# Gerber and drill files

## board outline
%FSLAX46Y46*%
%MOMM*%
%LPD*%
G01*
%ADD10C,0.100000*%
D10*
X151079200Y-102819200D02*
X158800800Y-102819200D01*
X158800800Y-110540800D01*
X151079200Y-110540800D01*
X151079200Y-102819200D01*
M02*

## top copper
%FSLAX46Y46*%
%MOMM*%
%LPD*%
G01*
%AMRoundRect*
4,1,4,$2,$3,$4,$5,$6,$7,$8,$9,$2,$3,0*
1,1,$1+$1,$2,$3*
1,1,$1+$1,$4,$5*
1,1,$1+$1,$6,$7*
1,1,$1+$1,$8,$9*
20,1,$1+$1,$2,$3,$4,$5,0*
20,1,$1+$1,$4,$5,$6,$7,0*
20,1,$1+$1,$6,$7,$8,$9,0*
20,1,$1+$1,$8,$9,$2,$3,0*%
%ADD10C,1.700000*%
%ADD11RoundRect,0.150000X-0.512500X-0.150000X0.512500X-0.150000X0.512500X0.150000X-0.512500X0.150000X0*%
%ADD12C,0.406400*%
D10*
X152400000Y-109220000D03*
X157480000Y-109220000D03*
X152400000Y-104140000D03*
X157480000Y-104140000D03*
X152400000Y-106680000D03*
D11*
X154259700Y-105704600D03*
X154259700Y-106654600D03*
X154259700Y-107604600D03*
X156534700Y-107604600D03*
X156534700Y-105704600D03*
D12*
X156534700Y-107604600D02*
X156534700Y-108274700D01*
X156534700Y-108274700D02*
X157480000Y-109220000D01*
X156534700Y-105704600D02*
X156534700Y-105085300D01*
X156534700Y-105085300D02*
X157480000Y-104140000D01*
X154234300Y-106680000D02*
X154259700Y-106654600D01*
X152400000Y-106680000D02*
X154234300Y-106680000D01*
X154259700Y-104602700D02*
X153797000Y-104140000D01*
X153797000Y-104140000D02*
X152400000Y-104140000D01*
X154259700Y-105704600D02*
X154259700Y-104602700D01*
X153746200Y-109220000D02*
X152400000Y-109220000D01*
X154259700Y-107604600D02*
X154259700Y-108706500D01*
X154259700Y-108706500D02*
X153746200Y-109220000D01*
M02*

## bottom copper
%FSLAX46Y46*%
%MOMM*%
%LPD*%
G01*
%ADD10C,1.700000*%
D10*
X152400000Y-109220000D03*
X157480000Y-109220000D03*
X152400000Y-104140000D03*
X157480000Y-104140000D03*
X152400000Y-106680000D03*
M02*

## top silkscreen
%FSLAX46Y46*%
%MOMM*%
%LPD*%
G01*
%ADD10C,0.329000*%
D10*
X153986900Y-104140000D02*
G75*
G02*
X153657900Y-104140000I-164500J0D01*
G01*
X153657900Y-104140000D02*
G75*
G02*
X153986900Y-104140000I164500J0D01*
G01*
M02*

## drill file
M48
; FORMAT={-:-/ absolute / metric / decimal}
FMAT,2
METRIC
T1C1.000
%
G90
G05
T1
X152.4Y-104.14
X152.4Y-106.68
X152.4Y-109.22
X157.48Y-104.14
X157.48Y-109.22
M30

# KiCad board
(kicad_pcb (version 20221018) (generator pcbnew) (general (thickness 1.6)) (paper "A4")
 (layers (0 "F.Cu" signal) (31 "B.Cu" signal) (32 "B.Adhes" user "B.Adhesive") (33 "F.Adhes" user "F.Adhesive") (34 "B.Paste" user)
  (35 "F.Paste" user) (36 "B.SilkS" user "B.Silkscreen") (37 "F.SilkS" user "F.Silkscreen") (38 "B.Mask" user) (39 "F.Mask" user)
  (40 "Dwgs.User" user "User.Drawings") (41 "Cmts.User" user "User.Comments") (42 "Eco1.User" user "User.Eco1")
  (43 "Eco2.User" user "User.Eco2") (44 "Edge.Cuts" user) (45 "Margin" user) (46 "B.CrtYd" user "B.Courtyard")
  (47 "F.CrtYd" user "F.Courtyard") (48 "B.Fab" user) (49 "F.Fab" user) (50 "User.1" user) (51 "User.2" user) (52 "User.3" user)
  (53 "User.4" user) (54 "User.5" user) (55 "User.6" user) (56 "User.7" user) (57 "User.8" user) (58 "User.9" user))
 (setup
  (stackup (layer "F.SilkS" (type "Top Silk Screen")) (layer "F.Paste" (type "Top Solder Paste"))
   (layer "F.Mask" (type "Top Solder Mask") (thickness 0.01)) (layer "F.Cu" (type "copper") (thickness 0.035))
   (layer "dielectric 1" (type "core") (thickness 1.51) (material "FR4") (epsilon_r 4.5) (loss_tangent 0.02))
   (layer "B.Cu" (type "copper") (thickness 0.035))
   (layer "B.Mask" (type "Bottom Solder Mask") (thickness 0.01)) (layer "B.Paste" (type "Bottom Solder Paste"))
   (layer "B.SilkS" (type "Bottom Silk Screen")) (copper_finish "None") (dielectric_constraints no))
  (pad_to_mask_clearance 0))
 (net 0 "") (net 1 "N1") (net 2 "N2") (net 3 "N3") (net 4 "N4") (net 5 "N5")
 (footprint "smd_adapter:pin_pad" (layer "F.Cu") (at 152.4 109.22)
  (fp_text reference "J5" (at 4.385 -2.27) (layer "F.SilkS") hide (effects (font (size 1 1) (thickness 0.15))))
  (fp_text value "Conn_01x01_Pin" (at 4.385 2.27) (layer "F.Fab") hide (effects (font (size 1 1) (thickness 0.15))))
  (pad "1" thru_hole circle (at 0 0) (size 1.7 1.7) (drill 1) (layers "*.Cu" "*.Mask") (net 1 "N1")))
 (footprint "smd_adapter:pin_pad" (layer "F.Cu") (at 157.48 109.22)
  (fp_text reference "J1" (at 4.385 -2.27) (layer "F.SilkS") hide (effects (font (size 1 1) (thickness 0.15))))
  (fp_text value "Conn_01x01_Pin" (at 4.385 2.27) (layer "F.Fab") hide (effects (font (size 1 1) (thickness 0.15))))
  (pad "1" thru_hole circle (at 0 0) (size 1.7 1.7) (drill 1) (layers "*.Cu" "*.Mask") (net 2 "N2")))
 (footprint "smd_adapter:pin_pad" (layer "F.Cu") (at 152.4 104.14)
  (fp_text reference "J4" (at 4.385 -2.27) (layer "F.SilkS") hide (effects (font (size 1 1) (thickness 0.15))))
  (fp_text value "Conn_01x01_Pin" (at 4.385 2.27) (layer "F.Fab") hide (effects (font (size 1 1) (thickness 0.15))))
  (pad "1" thru_hole circle (at 0 0) (size 1.7 1.7) (drill 1) (layers "*.Cu" "*.Mask") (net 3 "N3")))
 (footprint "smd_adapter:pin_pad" (layer "F.Cu") (at 157.48 104.14)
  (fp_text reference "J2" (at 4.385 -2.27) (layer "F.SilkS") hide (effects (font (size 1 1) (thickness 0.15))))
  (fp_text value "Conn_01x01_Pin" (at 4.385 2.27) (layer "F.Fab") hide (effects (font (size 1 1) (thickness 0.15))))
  (pad "1" thru_hole circle (at 0 0) (size 1.7 1.7) (drill 1) (layers "*.Cu" "*.Mask") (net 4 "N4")))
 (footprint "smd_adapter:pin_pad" (layer "F.Cu") (at 152.4 106.68)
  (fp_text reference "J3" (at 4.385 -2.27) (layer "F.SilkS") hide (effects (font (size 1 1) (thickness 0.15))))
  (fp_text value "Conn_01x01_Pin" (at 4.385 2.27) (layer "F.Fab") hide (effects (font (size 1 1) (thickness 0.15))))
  (pad "1" thru_hole circle (at 0 0) (size 1.7 1.7) (drill 1) (layers "*.Cu" "*.Mask") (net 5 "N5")))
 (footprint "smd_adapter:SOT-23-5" (layer "F.Cu") (at 155.3972 106.6546)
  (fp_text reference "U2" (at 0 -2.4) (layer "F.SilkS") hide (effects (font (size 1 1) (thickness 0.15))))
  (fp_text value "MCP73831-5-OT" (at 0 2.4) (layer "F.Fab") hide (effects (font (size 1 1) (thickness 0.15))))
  (pad "1" smd roundrect (at -1.1375 -0.95) (size 1.325 0.6) (layers "F.Cu" "F.Paste" "F.Mask") (roundrect_rratio 0.25) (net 3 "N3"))
  (pad "2" smd roundrect (at -1.1375 0) (size 1.325 0.6) (layers "F.Cu" "F.Paste" "F.Mask") (roundrect_rratio 0.25) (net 5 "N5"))
  (pad "3" smd roundrect (at -1.1375 0.95) (size 1.325 0.6) (layers "F.Cu" "F.Paste" "F.Mask") (roundrect_rratio 0.25) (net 1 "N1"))
  (pad "4" smd roundrect (at 1.1375 0.95) (size 1.325 0.6) (layers "F.Cu" "F.Paste" "F.Mask") (roundrect_rratio 0.25) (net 2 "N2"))
  (pad "5" smd roundrect (at 1.1375 -0.95) (size 1.325 0.6) (layers "F.Cu" "F.Paste" "F.Mask") (roundrect_rratio 0.25) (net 4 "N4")))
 (gr_circle (center 153.8224 104.14) (end 154.0764 104.14) (stroke (width 0.15) (type solid)) (fill solid) (layer "F.SilkS"))
 (gr_rect (start 151.0792 102.8192) (end 158.8008 110.5408) (stroke (width 0.1) (type default)) (fill none) (layer "Edge.Cuts"))
 (segment (start 156.5347 107.6046) (end 156.5347 108.2747) (width 0.4064) (layer "F.Cu") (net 2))
 (segment (start 156.5347 108.2747) (end 157.48 109.22) (width 0.4064) (layer "F.Cu") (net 2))
 (segment (start 156.5347 105.7046) (end 156.5347 105.0853) (width 0.4064) (layer "F.Cu") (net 4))
 (segment (start 156.5347 105.0853) (end 157.48 104.14) (width 0.4064) (layer "F.Cu") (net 4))
 (segment (start 154.2343 106.68) (end 154.2597 106.6546) (width 0.4064) (layer "F.Cu") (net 5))
 (segment (start 152.4 106.68) (end 154.2343 106.68) (width 0.4064) (layer "F.Cu") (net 5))
 (segment (start 154.2597 104.6027) (end 153.797 104.14) (width 0.4064) (layer "F.Cu") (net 3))
 (segment (start 153.797 104.14) (end 152.4 104.14) (width 0.4064) (layer "F.Cu") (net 3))
 (segment (start 154.2597 105.7046) (end 154.2597 104.6027) (width 0.4064) (layer "F.Cu") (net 3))
 (segment (start 153.7462 109.22) (end 152.4 109.22) (width 0.4064) (layer "F.Cu") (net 1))
 (segment (start 154.2597 107.6046) (end 154.2597 108.7065) (width 0.4064) (layer "F.Cu") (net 1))
 (segment (start 154.2597 108.7065) (end 153.7462 109.22) (width 0.4064) (layer "F.Cu") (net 1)))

